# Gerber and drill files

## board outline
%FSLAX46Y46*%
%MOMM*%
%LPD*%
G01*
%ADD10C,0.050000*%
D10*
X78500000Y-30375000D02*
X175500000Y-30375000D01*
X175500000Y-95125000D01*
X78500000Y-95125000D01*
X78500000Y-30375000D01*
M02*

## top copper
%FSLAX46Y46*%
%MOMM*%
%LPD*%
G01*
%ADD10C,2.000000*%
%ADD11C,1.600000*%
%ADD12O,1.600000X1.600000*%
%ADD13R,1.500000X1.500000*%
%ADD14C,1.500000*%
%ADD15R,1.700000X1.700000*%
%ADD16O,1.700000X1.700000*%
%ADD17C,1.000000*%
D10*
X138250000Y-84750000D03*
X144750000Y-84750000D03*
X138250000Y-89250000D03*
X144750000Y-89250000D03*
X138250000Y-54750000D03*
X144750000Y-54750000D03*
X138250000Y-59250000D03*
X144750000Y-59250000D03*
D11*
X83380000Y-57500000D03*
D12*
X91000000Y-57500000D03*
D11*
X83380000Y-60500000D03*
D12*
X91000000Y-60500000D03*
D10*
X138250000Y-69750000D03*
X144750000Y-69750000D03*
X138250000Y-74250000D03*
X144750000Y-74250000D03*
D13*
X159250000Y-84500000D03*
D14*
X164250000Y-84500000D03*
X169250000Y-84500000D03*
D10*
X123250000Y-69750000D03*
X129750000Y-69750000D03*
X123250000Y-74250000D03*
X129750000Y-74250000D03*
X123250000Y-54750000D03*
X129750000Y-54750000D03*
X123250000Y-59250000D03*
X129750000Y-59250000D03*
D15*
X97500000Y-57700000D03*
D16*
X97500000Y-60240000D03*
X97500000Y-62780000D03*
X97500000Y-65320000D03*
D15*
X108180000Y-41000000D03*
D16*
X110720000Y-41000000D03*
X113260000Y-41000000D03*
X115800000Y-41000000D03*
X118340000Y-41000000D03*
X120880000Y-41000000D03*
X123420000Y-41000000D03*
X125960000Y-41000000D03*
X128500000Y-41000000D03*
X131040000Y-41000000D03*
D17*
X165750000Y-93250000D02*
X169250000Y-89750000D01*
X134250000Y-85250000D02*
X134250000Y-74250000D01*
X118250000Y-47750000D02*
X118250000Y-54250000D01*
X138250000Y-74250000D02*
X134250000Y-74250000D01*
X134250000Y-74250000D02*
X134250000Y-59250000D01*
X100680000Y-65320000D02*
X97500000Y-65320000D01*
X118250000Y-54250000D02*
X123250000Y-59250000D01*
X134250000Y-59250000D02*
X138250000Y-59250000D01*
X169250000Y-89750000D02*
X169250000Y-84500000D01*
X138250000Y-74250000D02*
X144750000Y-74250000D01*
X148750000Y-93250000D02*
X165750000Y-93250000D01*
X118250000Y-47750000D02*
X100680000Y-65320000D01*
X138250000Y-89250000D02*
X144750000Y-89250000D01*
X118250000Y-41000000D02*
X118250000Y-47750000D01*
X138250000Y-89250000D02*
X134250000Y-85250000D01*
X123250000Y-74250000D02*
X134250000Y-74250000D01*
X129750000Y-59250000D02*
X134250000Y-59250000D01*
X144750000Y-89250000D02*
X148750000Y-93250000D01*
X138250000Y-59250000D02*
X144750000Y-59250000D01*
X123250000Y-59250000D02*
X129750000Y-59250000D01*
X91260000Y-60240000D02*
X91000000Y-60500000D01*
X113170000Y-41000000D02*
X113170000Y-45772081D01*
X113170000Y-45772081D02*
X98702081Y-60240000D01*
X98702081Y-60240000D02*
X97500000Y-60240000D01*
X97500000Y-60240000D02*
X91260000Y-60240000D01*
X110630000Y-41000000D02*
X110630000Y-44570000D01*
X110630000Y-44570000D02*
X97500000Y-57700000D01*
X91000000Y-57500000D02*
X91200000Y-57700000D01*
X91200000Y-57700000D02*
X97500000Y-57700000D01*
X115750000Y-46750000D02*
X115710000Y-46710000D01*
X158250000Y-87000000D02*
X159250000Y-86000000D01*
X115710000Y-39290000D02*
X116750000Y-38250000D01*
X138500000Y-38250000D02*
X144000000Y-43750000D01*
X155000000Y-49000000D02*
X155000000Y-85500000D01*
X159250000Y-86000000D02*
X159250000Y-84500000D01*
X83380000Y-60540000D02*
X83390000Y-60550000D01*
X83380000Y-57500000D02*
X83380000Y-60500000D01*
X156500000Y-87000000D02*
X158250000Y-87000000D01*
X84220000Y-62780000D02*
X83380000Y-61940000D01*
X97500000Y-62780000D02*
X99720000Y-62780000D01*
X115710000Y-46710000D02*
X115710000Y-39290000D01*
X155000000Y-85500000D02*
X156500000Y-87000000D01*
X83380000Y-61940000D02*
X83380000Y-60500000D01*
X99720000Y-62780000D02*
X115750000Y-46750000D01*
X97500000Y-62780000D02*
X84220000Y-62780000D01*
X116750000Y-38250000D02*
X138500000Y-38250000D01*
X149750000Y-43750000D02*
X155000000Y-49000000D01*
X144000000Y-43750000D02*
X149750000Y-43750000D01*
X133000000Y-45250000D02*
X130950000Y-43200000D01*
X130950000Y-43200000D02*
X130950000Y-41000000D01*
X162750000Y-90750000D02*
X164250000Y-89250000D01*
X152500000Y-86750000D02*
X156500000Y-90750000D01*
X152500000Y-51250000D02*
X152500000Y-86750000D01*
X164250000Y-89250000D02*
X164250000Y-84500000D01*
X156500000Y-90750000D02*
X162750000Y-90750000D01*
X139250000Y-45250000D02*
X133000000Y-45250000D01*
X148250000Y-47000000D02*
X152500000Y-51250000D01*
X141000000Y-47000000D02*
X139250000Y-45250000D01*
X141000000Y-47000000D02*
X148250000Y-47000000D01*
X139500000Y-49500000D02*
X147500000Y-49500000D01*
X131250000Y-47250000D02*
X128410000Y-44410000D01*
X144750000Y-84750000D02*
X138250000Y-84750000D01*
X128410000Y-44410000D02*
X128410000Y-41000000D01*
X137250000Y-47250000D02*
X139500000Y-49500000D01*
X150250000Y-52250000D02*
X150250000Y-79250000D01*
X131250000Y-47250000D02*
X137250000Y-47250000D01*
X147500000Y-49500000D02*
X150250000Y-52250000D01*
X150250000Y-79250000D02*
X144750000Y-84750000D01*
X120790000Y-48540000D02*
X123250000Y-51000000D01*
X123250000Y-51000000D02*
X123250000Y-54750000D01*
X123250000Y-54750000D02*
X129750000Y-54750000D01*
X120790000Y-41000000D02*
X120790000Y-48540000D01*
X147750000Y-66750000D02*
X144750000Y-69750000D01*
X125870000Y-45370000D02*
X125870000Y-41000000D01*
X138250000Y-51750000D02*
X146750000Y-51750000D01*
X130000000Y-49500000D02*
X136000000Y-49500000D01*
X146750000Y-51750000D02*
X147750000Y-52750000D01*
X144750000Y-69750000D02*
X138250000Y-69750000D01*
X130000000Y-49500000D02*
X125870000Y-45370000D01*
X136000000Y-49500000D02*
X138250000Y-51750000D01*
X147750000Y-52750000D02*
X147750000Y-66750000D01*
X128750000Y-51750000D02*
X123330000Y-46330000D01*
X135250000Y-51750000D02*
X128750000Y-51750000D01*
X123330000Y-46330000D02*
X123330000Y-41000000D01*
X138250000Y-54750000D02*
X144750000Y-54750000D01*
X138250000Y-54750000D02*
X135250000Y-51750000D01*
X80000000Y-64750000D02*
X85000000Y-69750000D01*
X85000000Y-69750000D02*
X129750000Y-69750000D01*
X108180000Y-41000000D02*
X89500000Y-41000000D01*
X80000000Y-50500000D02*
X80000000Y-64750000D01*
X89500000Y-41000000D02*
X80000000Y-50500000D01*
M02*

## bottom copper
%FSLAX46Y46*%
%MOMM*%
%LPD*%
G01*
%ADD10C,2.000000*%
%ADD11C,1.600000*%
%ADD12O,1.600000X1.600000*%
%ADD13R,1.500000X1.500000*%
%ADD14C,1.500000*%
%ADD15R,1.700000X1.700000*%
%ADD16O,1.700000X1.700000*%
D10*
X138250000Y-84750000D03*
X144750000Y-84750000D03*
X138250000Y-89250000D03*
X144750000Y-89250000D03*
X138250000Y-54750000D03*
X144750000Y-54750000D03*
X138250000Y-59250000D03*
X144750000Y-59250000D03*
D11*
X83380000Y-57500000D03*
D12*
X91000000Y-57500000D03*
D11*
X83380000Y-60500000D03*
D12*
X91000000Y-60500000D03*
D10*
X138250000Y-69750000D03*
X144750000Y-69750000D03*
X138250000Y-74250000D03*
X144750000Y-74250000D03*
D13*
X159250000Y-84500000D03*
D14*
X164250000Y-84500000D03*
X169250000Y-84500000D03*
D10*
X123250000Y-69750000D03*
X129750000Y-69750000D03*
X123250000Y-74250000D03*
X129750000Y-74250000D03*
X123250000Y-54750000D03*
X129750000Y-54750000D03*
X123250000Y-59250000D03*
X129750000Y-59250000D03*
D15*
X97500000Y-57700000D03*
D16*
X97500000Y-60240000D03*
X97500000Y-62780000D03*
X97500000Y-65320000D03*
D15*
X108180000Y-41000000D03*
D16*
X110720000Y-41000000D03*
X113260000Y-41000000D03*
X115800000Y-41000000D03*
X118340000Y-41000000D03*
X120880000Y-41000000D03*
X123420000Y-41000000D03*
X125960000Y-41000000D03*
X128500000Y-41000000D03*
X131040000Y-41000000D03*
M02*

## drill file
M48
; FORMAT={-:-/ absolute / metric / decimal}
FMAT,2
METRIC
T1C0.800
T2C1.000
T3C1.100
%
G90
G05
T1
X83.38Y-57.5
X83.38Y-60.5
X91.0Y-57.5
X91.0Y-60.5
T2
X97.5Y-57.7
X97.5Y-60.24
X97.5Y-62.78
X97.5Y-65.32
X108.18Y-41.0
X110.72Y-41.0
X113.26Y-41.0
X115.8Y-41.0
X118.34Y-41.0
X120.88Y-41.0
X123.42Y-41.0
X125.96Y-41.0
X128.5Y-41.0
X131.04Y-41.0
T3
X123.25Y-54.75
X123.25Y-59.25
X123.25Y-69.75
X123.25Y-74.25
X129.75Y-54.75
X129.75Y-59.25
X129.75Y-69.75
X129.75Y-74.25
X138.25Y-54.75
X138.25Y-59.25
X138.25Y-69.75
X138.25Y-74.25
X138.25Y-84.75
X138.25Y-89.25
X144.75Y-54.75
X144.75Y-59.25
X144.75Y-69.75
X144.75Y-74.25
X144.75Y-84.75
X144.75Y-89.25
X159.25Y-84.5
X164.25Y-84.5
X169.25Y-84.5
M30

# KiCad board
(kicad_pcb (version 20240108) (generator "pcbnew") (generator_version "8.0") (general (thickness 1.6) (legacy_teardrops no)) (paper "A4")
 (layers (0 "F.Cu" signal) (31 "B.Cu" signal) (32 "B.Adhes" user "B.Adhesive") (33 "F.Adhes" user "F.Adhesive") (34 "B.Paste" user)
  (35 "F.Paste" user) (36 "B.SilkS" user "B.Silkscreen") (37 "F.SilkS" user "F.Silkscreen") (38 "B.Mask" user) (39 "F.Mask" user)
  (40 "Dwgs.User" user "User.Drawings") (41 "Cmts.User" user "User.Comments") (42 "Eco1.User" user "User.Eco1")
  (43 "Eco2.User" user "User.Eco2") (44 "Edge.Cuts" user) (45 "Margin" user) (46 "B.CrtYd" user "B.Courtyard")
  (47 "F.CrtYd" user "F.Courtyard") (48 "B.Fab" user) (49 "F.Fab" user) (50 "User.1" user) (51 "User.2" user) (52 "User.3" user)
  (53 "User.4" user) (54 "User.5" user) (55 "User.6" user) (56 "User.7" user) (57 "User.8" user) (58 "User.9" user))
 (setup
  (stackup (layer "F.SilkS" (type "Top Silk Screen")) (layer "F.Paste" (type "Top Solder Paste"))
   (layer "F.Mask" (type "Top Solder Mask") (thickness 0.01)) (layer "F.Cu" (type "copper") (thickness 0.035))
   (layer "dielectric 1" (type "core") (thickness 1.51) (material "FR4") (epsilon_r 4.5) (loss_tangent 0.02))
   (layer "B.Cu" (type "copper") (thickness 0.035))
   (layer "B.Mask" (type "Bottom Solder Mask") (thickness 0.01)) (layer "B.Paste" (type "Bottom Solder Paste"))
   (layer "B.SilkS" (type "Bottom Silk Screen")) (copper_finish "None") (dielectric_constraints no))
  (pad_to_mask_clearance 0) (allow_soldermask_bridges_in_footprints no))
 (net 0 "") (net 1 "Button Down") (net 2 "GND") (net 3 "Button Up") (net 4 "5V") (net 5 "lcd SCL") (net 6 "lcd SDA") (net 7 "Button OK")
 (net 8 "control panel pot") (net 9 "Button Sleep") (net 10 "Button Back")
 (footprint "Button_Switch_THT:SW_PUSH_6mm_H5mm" (layer "F.Cu") (at 138.25 84.75)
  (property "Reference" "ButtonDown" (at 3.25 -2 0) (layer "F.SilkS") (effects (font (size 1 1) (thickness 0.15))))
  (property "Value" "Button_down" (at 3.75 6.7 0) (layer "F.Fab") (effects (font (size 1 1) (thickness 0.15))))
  (pad "1" thru_hole circle (at 0 0 90) (size 2 2) (drill 1.1) (layers "*.Cu" "*.Mask") (remove_unused_layers no) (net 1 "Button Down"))
  (pad "1" thru_hole circle (at 6.5 0 90) (size 2 2) (drill 1.1) (layers "*.Cu" "*.Mask") (remove_unused_layers no) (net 1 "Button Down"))
  (pad "2" thru_hole circle (at 0 4.5 90) (size 2 2) (drill 1.1) (layers "*.Cu" "*.Mask") (remove_unused_layers no) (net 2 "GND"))
  (pad "2" thru_hole circle (at 6.5 4.5 90) (size 2 2) (drill 1.1) (layers "*.Cu" "*.Mask") (remove_unused_layers no) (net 2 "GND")))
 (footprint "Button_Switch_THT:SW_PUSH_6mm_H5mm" (layer "F.Cu") (at 138.25 54.75)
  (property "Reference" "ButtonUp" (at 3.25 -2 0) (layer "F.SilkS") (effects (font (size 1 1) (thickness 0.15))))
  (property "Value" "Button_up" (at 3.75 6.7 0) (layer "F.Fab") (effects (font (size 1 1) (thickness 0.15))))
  (pad "1" thru_hole circle (at 0 0 90) (size 2 2) (drill 1.1) (layers "*.Cu" "*.Mask") (remove_unused_layers no) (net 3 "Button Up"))
  (pad "1" thru_hole circle (at 6.5 0 90) (size 2 2) (drill 1.1) (layers "*.Cu" "*.Mask") (remove_unused_layers no) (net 3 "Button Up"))
  (pad "2" thru_hole circle (at 0 4.5 90) (size 2 2) (drill 1.1) (layers "*.Cu" "*.Mask") (remove_unused_layers no) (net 2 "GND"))
  (pad "2" thru_hole circle (at 6.5 4.5 90) (size 2 2) (drill 1.1) (layers "*.Cu" "*.Mask") (remove_unused_layers no) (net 2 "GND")))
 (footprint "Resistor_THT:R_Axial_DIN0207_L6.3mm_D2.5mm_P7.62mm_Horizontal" (layer "F.Cu") (at 83.38 57.5)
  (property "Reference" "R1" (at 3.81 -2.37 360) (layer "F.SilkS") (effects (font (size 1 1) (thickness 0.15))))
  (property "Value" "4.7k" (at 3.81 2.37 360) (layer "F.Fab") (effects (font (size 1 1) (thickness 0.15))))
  (pad "1" thru_hole circle (at 0 0) (size 1.6 1.6) (drill 0.8) (layers "*.Cu" "*.Mask") (remove_unused_layers no) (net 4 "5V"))
  (pad "2" thru_hole oval (at 7.62 0) (size 1.6 1.6) (drill 0.8) (layers "*.Cu" "*.Mask") (remove_unused_layers no) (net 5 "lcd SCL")))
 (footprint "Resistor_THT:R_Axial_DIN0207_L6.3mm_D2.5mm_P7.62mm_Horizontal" (layer "F.Cu") (at 83.38 60.5)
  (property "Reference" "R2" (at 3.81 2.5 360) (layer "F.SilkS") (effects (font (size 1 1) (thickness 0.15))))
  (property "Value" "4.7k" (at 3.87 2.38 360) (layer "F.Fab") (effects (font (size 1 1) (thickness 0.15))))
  (pad "1" thru_hole circle (at 0 0) (size 1.6 1.6) (drill 0.8) (layers "*.Cu" "*.Mask") (remove_unused_layers no) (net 4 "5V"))
  (pad "2" thru_hole oval (at 7.62 0) (size 1.6 1.6) (drill 0.8) (layers "*.Cu" "*.Mask") (remove_unused_layers no) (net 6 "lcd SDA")))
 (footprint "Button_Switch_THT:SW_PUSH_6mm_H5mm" (layer "F.Cu") (at 138.25 69.75)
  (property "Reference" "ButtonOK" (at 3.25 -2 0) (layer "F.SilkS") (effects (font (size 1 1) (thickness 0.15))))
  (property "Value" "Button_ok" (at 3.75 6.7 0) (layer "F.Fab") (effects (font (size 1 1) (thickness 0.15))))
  (pad "1" thru_hole circle (at 0 0 90) (size 2 2) (drill 1.1) (layers "*.Cu" "*.Mask") (remove_unused_layers no) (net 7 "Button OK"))
  (pad "1" thru_hole circle (at 6.5 0 90) (size 2 2) (drill 1.1) (layers "*.Cu" "*.Mask") (remove_unused_layers no) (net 7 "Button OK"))
  (pad "2" thru_hole circle (at 0 4.5 90) (size 2 2) (drill 1.1) (layers "*.Cu" "*.Mask") (remove_unused_layers no) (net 2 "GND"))
  (pad "2" thru_hole circle (at 6.5 4.5 90) (size 2 2) (drill 1.1) (layers "*.Cu" "*.Mask") (remove_unused_layers no) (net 2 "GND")))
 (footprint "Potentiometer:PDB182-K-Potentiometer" (layer "F.Cu") (at 164.25 84.5)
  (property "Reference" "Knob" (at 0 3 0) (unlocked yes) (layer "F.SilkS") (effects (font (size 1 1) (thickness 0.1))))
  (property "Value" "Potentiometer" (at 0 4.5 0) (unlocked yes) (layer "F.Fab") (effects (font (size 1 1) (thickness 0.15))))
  (pad "1" thru_hole rect (at -5 0) (size 1.5 1.5) (drill 1.1) (layers "*.Cu" "*.Mask") (remove_unused_layers no) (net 4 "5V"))
  (pad "2" thru_hole circle (at 0 0) (size 1.5 1.5) (drill 1.1) (layers "*.Cu" "*.Mask") (remove_unused_layers no)
   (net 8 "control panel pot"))
  (pad "3" thru_hole circle (at 5 0) (size 1.5 1.5) (drill 1.1) (layers "*.Cu" "*.Mask") (remove_unused_layers no) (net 2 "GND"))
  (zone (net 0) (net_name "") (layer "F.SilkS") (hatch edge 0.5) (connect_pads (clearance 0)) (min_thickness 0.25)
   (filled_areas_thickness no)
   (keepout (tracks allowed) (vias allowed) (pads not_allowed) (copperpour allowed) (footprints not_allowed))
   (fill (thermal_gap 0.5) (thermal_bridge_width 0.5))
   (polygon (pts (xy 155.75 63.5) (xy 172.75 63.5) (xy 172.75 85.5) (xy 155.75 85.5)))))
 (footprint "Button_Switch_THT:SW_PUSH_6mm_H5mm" (layer "F.Cu") (at 123.25 69.75)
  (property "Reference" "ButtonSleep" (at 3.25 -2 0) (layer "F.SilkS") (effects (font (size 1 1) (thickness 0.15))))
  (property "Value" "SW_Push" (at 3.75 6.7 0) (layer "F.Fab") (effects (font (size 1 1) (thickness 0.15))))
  (pad "1" thru_hole circle (at 0 0 90) (size 2 2) (drill 1.1) (layers "*.Cu" "*.Mask") (remove_unused_layers no) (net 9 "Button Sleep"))
  (pad "1" thru_hole circle (at 6.5 0 90) (size 2 2) (drill 1.1) (layers "*.Cu" "*.Mask") (remove_unused_layers no) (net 9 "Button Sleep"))
  (pad "2" thru_hole circle (at 0 4.5 90) (size 2 2) (drill 1.1) (layers "*.Cu" "*.Mask") (remove_unused_layers no) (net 2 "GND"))
  (pad "2" thru_hole circle (at 6.5 4.5 90) (size 2 2) (drill 1.1) (layers "*.Cu" "*.Mask") (remove_unused_layers no) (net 2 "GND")))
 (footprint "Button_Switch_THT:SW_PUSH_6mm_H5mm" (layer "F.Cu") (at 123.25 54.75)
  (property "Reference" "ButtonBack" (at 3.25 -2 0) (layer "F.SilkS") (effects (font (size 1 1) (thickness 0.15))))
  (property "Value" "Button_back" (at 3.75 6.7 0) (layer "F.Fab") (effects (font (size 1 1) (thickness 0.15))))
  (pad "1" thru_hole circle (at 0 0 90) (size 2 2) (drill 1.1) (layers "*.Cu" "*.Mask") (remove_unused_layers no) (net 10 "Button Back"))
  (pad "1" thru_hole circle (at 6.5 0 90) (size 2 2) (drill 1.1) (layers "*.Cu" "*.Mask") (remove_unused_layers no) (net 10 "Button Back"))
  (pad "2" thru_hole circle (at 0 4.5 90) (size 2 2) (drill 1.1) (layers "*.Cu" "*.Mask") (remove_unused_layers no) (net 2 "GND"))
  (pad "2" thru_hole circle (at 6.5 4.5 90) (size 2 2) (drill 1.1) (layers "*.Cu" "*.Mask") (remove_unused_layers no) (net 2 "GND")))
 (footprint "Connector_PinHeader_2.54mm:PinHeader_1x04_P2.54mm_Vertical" (layer "F.Cu") (at 97.5 57.7)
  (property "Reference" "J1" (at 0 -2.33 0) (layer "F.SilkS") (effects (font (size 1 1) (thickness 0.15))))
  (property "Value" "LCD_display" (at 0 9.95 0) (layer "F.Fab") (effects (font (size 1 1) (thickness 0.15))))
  (pad "1" thru_hole rect (at 0 0) (size 1.7 1.7) (drill 1) (layers "*.Cu" "*.Mask") (remove_unused_layers no) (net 5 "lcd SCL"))
  (pad "2" thru_hole oval (at 0 2.54) (size 1.7 1.7) (drill 1) (layers "*.Cu" "*.Mask") (remove_unused_layers no) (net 6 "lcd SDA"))
  (pad "3" thru_hole oval (at 0 5.08) (size 1.7 1.7) (drill 1) (layers "*.Cu" "*.Mask") (remove_unused_layers no) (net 4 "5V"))
  (pad "4" thru_hole oval (at 0 7.62) (size 1.7 1.7) (drill 1) (layers "*.Cu" "*.Mask") (remove_unused_layers no) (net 2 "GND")))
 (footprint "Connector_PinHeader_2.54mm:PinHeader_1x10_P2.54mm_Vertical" (layer "F.Cu") (at 108.18 41 90)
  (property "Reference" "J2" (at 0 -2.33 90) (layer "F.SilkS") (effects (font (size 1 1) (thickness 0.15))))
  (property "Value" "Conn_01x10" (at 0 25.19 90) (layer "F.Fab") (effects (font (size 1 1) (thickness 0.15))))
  (pad "1" thru_hole rect (at 0 0 90) (size 1.7 1.7) (drill 1) (layers "*.Cu" "*.Mask") (remove_unused_layers no) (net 9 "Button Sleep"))
  (pad "2" thru_hole oval (at 0 2.54 90) (size 1.7 1.7) (drill 1) (layers "*.Cu" "*.Mask") (remove_unused_layers no) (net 5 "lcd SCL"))
  (pad "3" thru_hole oval (at 0 5.08 90) (size 1.7 1.7) (drill 1) (layers "*.Cu" "*.Mask") (remove_unused_layers no) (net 6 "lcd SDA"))
  (pad "4" thru_hole oval (at 0 7.62 90) (size 1.7 1.7) (drill 1) (layers "*.Cu" "*.Mask") (remove_unused_layers no) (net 4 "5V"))
  (pad "5" thru_hole oval (at 0 10.16 90) (size 1.7 1.7) (drill 1) (layers "*.Cu" "*.Mask") (remove_unused_layers no) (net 2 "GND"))
  (pad "6" thru_hole oval (at 0 12.7 90) (size 1.7 1.7) (drill 1) (layers "*.Cu" "*.Mask") (remove_unused_layers no) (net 10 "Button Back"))
  (pad "7" thru_hole oval (at 0 15.24 90) (size 1.7 1.7) (drill 1) (layers "*.Cu" "*.Mask") (remove_unused_layers no) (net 3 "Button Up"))
  (pad "8" thru_hole oval (at 0 17.78 90) (size 1.7 1.7) (drill 1) (layers "*.Cu" "*.Mask") (remove_unused_layers no) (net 7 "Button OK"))
  (pad "9" thru_hole oval (at 0 20.32 90) (size 1.7 1.7) (drill 1) (layers "*.Cu" "*.Mask") (remove_unused_layers no) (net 1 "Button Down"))
  (pad "10" thru_hole oval (at 0 22.86 90) (size 1.7 1.7) (drill 1) (layers "*.Cu" "*.Mask") (remove_unused_layers no)
   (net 8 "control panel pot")))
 (gr_rect (start 78.5 30.375) (end 175.5 95.125) (stroke (width 0.05) (type default)) (fill none) (layer "Edge.Cuts"))
 (segment (start 165.75 93.25) (end 169.25 89.75) (width 1) (layer "F.Cu") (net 2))
 (segment (start 134.25 85.25) (end 134.25 74.25) (width 1) (layer "F.Cu") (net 2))
 (segment (start 118.25 47.75) (end 118.25 54.25) (width 1) (layer "F.Cu") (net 2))
 (segment (start 138.25 74.25) (end 134.25 74.25) (width 1) (layer "F.Cu") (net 2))
 (segment (start 134.25 74.25) (end 134.25 59.25) (width 1) (layer "F.Cu") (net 2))
 (segment (start 100.68 65.32) (end 97.5 65.32) (width 1) (layer "F.Cu") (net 2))
 (segment (start 118.25 54.25) (end 123.25 59.25) (width 1) (layer "F.Cu") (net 2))
 (segment (start 134.25 59.25) (end 138.25 59.25) (width 1) (layer "F.Cu") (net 2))
 (segment (start 169.25 89.75) (end 169.25 84.5) (width 1) (layer "F.Cu") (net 2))
 (segment (start 138.25 74.25) (end 144.75 74.25) (width 1) (layer "F.Cu") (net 2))
 (segment (start 148.75 93.25) (end 165.75 93.25) (width 1) (layer "F.Cu") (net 2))
 (segment (start 118.25 47.75) (end 100.68 65.32) (width 1) (layer "F.Cu") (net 2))
 (segment (start 138.25 89.25) (end 144.75 89.25) (width 1) (layer "F.Cu") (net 2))
 (segment (start 118.25 41) (end 118.25 47.75) (width 1) (layer "F.Cu") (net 2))
 (segment (start 138.25 89.25) (end 134.25 85.25) (width 1) (layer "F.Cu") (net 2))
 (segment (start 123.25 74.25) (end 134.25 74.25) (width 1) (layer "F.Cu") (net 2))
 (segment (start 129.75 59.25) (end 134.25 59.25) (width 1) (layer "F.Cu") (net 2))
 (segment (start 144.75 89.25) (end 148.75 93.25) (width 1) (layer "F.Cu") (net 2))
 (segment (start 138.25 59.25) (end 144.75 59.25) (width 1) (layer "F.Cu") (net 2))
 (segment (start 123.25 59.25) (end 129.75 59.25) (width 1) (layer "F.Cu") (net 2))
 (segment (start 91.26 60.24) (end 91 60.5) (width 1) (layer "F.Cu") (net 6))
 (segment (start 113.17 41) (end 113.17 45.772081) (width 1) (layer "F.Cu") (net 6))
 (segment (start 113.17 45.772081) (end 98.702081 60.24) (width 1) (layer "F.Cu") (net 6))
 (segment (start 98.702081 60.24) (end 97.5 60.24) (width 1) (layer "F.Cu") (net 6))
 (segment (start 97.5 60.24) (end 91.26 60.24) (width 1) (layer "F.Cu") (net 6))
 (segment (start 110.63 41) (end 110.63 44.57) (width 1) (layer "F.Cu") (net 5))
 (segment (start 110.63 44.57) (end 97.5 57.7) (width 1) (layer "F.Cu") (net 5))
 (segment (start 91 57.5) (end 91.2 57.7) (width 1) (layer "F.Cu") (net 5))
 (segment (start 91.2 57.7) (end 97.5 57.7) (width 1) (layer "F.Cu") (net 5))
 (segment (start 115.75 46.75) (end 115.71 46.71) (width 1) (layer "F.Cu") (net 4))
 (segment (start 158.25 87) (end 159.25 86) (width 1) (layer "F.Cu") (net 4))
 (segment (start 115.71 39.29) (end 116.75 38.25) (width 1) (layer "F.Cu") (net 4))
 (segment (start 138.5 38.25) (end 144 43.75) (width 1) (layer "F.Cu") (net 4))
 (segment (start 155 49) (end 155 85.5) (width 1) (layer "F.Cu") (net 4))
 (segment (start 159.25 86) (end 159.25 84.5) (width 1) (layer "F.Cu") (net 4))
 (segment (start 83.38 60.54) (end 83.39 60.55) (width 1) (layer "F.Cu") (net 4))
 (segment (start 83.38 57.5) (end 83.38 60.5) (width 1) (layer "F.Cu") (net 4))
 (segment (start 156.5 87) (end 158.25 87) (width 1) (layer "F.Cu") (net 4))
 (segment (start 84.22 62.78) (end 83.38 61.94) (width 1) (layer "F.Cu") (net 4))
 (segment (start 97.5 62.78) (end 99.72 62.78) (width 1) (layer "F.Cu") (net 4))
 (segment (start 115.71 46.71) (end 115.71 39.29) (width 1) (layer "F.Cu") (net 4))
 (segment (start 155 85.5) (end 156.5 87) (width 1) (layer "F.Cu") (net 4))
 (segment (start 83.38 61.94) (end 83.38 60.5) (width 1) (layer "F.Cu") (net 4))
 (segment (start 99.72 62.78) (end 115.75 46.75) (width 1) (layer "F.Cu") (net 4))
 (segment (start 97.5 62.78) (end 84.22 62.78) (width 1) (layer "F.Cu") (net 4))
 (segment (start 116.75 38.25) (end 138.5 38.25) (width 1) (layer "F.Cu") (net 4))
 (segment (start 149.75 43.75) (end 155 49) (width 1) (layer "F.Cu") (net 4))
 (segment (start 144 43.75) (end 149.75 43.75) (width 1) (layer "F.Cu") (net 4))
 (segment (start 133 45.25) (end 130.95 43.2) (width 1) (layer "F.Cu") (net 8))
 (segment (start 130.95 43.2) (end 130.95 41) (width 1) (layer "F.Cu") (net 8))
 (segment (start 162.75 90.75) (end 164.25 89.25) (width 1) (layer "F.Cu") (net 8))
 (segment (start 152.5 86.75) (end 156.5 90.75) (width 1) (layer "F.Cu") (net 8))
 (segment (start 152.5 51.25) (end 152.5 86.75) (width 1) (layer "F.Cu") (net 8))
 (segment (start 164.25 89.25) (end 164.25 84.5) (width 1) (layer "F.Cu") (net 8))
 (segment (start 156.5 90.75) (end 162.75 90.75) (width 1) (layer "F.Cu") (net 8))
 (segment (start 139.25 45.25) (end 133 45.25) (width 1) (layer "F.Cu") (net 8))
 (segment (start 148.25 47) (end 152.5 51.25) (width 1) (layer "F.Cu") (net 8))
 (segment (start 141 47) (end 139.25 45.25) (width 1) (layer "F.Cu") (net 8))
 (segment (start 141 47) (end 148.25 47) (width 1) (layer "F.Cu") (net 8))
 (segment (start 139.5 49.5) (end 147.5 49.5) (width 1) (layer "F.Cu") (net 1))
 (segment (start 131.25 47.25) (end 128.41 44.41) (width 1) (layer "F.Cu") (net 1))
 (segment (start 144.75 84.75) (end 138.25 84.75) (width 1) (layer "F.Cu") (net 1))
 (segment (start 128.41 44.41) (end 128.41 41) (width 1) (layer "F.Cu") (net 1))
 (segment (start 137.25 47.25) (end 139.5 49.5) (width 1) (layer "F.Cu") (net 1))
 (segment (start 150.25 52.25) (end 150.25 79.25) (width 1) (layer "F.Cu") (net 1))
 (segment (start 131.25 47.25) (end 137.25 47.25) (width 1) (layer "F.Cu") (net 1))
 (segment (start 147.5 49.5) (end 150.25 52.25) (width 1) (layer "F.Cu") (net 1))
 (segment (start 150.25 79.25) (end 144.75 84.75) (width 1) (layer "F.Cu") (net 1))
 (segment (start 120.79 48.54) (end 123.25 51) (width 1) (layer "F.Cu") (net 10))
 (segment (start 123.25 51) (end 123.25 54.75) (width 1) (layer "F.Cu") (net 10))
 (segment (start 123.25 54.75) (end 129.75 54.75) (width 1) (layer "F.Cu") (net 10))
 (segment (start 120.79 41) (end 120.79 48.54) (width 1) (layer "F.Cu") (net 10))
 (segment (start 147.75 66.75) (end 144.75 69.75) (width 1) (layer "F.Cu") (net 7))
 (segment (start 125.87 45.37) (end 125.87 41) (width 1) (layer "F.Cu") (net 7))
 (segment (start 138.25 51.75) (end 146.75 51.75) (width 1) (layer "F.Cu") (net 7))
 (segment (start 130 49.5) (end 136 49.5) (width 1) (layer "F.Cu") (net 7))
 (segment (start 146.75 51.75) (end 147.75 52.75) (width 1) (layer "F.Cu") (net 7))
 (segment (start 144.75 69.75) (end 138.25 69.75) (width 1) (layer "F.Cu") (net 7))
 (segment (start 130 49.5) (end 125.87 45.37) (width 1) (layer "F.Cu") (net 7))
 (segment (start 136 49.5) (end 138.25 51.75) (width 1) (layer "F.Cu") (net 7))
 (segment (start 147.75 52.75) (end 147.75 66.75) (width 1) (layer "F.Cu") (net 7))
 (segment (start 128.75 51.75) (end 123.33 46.33) (width 1) (layer "F.Cu") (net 3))
 (segment (start 135.25 51.75) (end 128.75 51.75) (width 1) (layer "F.Cu") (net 3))
 (segment (start 123.33 46.33) (end 123.33 41) (width 1) (layer "F.Cu") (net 3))
 (segment (start 138.25 54.75) (end 144.75 54.75) (width 1) (layer "F.Cu") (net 3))
 (segment (start 138.25 54.75) (end 135.25 51.75) (width 1) (layer "F.Cu") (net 3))
 (segment (start 80 64.75) (end 85 69.75) (width 1) (layer "F.Cu") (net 9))
 (segment (start 85 69.75) (end 129.75 69.75) (width 1) (layer "F.Cu") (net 9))
 (segment (start 108.18 41) (end 89.5 41) (width 1) (layer "F.Cu") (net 9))
 (segment (start 80 50.5) (end 80 64.75) (width 1) (layer "F.Cu") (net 9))
 (segment (start 89.5 41) (end 80 50.5) (width 1) (layer "F.Cu") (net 9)))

